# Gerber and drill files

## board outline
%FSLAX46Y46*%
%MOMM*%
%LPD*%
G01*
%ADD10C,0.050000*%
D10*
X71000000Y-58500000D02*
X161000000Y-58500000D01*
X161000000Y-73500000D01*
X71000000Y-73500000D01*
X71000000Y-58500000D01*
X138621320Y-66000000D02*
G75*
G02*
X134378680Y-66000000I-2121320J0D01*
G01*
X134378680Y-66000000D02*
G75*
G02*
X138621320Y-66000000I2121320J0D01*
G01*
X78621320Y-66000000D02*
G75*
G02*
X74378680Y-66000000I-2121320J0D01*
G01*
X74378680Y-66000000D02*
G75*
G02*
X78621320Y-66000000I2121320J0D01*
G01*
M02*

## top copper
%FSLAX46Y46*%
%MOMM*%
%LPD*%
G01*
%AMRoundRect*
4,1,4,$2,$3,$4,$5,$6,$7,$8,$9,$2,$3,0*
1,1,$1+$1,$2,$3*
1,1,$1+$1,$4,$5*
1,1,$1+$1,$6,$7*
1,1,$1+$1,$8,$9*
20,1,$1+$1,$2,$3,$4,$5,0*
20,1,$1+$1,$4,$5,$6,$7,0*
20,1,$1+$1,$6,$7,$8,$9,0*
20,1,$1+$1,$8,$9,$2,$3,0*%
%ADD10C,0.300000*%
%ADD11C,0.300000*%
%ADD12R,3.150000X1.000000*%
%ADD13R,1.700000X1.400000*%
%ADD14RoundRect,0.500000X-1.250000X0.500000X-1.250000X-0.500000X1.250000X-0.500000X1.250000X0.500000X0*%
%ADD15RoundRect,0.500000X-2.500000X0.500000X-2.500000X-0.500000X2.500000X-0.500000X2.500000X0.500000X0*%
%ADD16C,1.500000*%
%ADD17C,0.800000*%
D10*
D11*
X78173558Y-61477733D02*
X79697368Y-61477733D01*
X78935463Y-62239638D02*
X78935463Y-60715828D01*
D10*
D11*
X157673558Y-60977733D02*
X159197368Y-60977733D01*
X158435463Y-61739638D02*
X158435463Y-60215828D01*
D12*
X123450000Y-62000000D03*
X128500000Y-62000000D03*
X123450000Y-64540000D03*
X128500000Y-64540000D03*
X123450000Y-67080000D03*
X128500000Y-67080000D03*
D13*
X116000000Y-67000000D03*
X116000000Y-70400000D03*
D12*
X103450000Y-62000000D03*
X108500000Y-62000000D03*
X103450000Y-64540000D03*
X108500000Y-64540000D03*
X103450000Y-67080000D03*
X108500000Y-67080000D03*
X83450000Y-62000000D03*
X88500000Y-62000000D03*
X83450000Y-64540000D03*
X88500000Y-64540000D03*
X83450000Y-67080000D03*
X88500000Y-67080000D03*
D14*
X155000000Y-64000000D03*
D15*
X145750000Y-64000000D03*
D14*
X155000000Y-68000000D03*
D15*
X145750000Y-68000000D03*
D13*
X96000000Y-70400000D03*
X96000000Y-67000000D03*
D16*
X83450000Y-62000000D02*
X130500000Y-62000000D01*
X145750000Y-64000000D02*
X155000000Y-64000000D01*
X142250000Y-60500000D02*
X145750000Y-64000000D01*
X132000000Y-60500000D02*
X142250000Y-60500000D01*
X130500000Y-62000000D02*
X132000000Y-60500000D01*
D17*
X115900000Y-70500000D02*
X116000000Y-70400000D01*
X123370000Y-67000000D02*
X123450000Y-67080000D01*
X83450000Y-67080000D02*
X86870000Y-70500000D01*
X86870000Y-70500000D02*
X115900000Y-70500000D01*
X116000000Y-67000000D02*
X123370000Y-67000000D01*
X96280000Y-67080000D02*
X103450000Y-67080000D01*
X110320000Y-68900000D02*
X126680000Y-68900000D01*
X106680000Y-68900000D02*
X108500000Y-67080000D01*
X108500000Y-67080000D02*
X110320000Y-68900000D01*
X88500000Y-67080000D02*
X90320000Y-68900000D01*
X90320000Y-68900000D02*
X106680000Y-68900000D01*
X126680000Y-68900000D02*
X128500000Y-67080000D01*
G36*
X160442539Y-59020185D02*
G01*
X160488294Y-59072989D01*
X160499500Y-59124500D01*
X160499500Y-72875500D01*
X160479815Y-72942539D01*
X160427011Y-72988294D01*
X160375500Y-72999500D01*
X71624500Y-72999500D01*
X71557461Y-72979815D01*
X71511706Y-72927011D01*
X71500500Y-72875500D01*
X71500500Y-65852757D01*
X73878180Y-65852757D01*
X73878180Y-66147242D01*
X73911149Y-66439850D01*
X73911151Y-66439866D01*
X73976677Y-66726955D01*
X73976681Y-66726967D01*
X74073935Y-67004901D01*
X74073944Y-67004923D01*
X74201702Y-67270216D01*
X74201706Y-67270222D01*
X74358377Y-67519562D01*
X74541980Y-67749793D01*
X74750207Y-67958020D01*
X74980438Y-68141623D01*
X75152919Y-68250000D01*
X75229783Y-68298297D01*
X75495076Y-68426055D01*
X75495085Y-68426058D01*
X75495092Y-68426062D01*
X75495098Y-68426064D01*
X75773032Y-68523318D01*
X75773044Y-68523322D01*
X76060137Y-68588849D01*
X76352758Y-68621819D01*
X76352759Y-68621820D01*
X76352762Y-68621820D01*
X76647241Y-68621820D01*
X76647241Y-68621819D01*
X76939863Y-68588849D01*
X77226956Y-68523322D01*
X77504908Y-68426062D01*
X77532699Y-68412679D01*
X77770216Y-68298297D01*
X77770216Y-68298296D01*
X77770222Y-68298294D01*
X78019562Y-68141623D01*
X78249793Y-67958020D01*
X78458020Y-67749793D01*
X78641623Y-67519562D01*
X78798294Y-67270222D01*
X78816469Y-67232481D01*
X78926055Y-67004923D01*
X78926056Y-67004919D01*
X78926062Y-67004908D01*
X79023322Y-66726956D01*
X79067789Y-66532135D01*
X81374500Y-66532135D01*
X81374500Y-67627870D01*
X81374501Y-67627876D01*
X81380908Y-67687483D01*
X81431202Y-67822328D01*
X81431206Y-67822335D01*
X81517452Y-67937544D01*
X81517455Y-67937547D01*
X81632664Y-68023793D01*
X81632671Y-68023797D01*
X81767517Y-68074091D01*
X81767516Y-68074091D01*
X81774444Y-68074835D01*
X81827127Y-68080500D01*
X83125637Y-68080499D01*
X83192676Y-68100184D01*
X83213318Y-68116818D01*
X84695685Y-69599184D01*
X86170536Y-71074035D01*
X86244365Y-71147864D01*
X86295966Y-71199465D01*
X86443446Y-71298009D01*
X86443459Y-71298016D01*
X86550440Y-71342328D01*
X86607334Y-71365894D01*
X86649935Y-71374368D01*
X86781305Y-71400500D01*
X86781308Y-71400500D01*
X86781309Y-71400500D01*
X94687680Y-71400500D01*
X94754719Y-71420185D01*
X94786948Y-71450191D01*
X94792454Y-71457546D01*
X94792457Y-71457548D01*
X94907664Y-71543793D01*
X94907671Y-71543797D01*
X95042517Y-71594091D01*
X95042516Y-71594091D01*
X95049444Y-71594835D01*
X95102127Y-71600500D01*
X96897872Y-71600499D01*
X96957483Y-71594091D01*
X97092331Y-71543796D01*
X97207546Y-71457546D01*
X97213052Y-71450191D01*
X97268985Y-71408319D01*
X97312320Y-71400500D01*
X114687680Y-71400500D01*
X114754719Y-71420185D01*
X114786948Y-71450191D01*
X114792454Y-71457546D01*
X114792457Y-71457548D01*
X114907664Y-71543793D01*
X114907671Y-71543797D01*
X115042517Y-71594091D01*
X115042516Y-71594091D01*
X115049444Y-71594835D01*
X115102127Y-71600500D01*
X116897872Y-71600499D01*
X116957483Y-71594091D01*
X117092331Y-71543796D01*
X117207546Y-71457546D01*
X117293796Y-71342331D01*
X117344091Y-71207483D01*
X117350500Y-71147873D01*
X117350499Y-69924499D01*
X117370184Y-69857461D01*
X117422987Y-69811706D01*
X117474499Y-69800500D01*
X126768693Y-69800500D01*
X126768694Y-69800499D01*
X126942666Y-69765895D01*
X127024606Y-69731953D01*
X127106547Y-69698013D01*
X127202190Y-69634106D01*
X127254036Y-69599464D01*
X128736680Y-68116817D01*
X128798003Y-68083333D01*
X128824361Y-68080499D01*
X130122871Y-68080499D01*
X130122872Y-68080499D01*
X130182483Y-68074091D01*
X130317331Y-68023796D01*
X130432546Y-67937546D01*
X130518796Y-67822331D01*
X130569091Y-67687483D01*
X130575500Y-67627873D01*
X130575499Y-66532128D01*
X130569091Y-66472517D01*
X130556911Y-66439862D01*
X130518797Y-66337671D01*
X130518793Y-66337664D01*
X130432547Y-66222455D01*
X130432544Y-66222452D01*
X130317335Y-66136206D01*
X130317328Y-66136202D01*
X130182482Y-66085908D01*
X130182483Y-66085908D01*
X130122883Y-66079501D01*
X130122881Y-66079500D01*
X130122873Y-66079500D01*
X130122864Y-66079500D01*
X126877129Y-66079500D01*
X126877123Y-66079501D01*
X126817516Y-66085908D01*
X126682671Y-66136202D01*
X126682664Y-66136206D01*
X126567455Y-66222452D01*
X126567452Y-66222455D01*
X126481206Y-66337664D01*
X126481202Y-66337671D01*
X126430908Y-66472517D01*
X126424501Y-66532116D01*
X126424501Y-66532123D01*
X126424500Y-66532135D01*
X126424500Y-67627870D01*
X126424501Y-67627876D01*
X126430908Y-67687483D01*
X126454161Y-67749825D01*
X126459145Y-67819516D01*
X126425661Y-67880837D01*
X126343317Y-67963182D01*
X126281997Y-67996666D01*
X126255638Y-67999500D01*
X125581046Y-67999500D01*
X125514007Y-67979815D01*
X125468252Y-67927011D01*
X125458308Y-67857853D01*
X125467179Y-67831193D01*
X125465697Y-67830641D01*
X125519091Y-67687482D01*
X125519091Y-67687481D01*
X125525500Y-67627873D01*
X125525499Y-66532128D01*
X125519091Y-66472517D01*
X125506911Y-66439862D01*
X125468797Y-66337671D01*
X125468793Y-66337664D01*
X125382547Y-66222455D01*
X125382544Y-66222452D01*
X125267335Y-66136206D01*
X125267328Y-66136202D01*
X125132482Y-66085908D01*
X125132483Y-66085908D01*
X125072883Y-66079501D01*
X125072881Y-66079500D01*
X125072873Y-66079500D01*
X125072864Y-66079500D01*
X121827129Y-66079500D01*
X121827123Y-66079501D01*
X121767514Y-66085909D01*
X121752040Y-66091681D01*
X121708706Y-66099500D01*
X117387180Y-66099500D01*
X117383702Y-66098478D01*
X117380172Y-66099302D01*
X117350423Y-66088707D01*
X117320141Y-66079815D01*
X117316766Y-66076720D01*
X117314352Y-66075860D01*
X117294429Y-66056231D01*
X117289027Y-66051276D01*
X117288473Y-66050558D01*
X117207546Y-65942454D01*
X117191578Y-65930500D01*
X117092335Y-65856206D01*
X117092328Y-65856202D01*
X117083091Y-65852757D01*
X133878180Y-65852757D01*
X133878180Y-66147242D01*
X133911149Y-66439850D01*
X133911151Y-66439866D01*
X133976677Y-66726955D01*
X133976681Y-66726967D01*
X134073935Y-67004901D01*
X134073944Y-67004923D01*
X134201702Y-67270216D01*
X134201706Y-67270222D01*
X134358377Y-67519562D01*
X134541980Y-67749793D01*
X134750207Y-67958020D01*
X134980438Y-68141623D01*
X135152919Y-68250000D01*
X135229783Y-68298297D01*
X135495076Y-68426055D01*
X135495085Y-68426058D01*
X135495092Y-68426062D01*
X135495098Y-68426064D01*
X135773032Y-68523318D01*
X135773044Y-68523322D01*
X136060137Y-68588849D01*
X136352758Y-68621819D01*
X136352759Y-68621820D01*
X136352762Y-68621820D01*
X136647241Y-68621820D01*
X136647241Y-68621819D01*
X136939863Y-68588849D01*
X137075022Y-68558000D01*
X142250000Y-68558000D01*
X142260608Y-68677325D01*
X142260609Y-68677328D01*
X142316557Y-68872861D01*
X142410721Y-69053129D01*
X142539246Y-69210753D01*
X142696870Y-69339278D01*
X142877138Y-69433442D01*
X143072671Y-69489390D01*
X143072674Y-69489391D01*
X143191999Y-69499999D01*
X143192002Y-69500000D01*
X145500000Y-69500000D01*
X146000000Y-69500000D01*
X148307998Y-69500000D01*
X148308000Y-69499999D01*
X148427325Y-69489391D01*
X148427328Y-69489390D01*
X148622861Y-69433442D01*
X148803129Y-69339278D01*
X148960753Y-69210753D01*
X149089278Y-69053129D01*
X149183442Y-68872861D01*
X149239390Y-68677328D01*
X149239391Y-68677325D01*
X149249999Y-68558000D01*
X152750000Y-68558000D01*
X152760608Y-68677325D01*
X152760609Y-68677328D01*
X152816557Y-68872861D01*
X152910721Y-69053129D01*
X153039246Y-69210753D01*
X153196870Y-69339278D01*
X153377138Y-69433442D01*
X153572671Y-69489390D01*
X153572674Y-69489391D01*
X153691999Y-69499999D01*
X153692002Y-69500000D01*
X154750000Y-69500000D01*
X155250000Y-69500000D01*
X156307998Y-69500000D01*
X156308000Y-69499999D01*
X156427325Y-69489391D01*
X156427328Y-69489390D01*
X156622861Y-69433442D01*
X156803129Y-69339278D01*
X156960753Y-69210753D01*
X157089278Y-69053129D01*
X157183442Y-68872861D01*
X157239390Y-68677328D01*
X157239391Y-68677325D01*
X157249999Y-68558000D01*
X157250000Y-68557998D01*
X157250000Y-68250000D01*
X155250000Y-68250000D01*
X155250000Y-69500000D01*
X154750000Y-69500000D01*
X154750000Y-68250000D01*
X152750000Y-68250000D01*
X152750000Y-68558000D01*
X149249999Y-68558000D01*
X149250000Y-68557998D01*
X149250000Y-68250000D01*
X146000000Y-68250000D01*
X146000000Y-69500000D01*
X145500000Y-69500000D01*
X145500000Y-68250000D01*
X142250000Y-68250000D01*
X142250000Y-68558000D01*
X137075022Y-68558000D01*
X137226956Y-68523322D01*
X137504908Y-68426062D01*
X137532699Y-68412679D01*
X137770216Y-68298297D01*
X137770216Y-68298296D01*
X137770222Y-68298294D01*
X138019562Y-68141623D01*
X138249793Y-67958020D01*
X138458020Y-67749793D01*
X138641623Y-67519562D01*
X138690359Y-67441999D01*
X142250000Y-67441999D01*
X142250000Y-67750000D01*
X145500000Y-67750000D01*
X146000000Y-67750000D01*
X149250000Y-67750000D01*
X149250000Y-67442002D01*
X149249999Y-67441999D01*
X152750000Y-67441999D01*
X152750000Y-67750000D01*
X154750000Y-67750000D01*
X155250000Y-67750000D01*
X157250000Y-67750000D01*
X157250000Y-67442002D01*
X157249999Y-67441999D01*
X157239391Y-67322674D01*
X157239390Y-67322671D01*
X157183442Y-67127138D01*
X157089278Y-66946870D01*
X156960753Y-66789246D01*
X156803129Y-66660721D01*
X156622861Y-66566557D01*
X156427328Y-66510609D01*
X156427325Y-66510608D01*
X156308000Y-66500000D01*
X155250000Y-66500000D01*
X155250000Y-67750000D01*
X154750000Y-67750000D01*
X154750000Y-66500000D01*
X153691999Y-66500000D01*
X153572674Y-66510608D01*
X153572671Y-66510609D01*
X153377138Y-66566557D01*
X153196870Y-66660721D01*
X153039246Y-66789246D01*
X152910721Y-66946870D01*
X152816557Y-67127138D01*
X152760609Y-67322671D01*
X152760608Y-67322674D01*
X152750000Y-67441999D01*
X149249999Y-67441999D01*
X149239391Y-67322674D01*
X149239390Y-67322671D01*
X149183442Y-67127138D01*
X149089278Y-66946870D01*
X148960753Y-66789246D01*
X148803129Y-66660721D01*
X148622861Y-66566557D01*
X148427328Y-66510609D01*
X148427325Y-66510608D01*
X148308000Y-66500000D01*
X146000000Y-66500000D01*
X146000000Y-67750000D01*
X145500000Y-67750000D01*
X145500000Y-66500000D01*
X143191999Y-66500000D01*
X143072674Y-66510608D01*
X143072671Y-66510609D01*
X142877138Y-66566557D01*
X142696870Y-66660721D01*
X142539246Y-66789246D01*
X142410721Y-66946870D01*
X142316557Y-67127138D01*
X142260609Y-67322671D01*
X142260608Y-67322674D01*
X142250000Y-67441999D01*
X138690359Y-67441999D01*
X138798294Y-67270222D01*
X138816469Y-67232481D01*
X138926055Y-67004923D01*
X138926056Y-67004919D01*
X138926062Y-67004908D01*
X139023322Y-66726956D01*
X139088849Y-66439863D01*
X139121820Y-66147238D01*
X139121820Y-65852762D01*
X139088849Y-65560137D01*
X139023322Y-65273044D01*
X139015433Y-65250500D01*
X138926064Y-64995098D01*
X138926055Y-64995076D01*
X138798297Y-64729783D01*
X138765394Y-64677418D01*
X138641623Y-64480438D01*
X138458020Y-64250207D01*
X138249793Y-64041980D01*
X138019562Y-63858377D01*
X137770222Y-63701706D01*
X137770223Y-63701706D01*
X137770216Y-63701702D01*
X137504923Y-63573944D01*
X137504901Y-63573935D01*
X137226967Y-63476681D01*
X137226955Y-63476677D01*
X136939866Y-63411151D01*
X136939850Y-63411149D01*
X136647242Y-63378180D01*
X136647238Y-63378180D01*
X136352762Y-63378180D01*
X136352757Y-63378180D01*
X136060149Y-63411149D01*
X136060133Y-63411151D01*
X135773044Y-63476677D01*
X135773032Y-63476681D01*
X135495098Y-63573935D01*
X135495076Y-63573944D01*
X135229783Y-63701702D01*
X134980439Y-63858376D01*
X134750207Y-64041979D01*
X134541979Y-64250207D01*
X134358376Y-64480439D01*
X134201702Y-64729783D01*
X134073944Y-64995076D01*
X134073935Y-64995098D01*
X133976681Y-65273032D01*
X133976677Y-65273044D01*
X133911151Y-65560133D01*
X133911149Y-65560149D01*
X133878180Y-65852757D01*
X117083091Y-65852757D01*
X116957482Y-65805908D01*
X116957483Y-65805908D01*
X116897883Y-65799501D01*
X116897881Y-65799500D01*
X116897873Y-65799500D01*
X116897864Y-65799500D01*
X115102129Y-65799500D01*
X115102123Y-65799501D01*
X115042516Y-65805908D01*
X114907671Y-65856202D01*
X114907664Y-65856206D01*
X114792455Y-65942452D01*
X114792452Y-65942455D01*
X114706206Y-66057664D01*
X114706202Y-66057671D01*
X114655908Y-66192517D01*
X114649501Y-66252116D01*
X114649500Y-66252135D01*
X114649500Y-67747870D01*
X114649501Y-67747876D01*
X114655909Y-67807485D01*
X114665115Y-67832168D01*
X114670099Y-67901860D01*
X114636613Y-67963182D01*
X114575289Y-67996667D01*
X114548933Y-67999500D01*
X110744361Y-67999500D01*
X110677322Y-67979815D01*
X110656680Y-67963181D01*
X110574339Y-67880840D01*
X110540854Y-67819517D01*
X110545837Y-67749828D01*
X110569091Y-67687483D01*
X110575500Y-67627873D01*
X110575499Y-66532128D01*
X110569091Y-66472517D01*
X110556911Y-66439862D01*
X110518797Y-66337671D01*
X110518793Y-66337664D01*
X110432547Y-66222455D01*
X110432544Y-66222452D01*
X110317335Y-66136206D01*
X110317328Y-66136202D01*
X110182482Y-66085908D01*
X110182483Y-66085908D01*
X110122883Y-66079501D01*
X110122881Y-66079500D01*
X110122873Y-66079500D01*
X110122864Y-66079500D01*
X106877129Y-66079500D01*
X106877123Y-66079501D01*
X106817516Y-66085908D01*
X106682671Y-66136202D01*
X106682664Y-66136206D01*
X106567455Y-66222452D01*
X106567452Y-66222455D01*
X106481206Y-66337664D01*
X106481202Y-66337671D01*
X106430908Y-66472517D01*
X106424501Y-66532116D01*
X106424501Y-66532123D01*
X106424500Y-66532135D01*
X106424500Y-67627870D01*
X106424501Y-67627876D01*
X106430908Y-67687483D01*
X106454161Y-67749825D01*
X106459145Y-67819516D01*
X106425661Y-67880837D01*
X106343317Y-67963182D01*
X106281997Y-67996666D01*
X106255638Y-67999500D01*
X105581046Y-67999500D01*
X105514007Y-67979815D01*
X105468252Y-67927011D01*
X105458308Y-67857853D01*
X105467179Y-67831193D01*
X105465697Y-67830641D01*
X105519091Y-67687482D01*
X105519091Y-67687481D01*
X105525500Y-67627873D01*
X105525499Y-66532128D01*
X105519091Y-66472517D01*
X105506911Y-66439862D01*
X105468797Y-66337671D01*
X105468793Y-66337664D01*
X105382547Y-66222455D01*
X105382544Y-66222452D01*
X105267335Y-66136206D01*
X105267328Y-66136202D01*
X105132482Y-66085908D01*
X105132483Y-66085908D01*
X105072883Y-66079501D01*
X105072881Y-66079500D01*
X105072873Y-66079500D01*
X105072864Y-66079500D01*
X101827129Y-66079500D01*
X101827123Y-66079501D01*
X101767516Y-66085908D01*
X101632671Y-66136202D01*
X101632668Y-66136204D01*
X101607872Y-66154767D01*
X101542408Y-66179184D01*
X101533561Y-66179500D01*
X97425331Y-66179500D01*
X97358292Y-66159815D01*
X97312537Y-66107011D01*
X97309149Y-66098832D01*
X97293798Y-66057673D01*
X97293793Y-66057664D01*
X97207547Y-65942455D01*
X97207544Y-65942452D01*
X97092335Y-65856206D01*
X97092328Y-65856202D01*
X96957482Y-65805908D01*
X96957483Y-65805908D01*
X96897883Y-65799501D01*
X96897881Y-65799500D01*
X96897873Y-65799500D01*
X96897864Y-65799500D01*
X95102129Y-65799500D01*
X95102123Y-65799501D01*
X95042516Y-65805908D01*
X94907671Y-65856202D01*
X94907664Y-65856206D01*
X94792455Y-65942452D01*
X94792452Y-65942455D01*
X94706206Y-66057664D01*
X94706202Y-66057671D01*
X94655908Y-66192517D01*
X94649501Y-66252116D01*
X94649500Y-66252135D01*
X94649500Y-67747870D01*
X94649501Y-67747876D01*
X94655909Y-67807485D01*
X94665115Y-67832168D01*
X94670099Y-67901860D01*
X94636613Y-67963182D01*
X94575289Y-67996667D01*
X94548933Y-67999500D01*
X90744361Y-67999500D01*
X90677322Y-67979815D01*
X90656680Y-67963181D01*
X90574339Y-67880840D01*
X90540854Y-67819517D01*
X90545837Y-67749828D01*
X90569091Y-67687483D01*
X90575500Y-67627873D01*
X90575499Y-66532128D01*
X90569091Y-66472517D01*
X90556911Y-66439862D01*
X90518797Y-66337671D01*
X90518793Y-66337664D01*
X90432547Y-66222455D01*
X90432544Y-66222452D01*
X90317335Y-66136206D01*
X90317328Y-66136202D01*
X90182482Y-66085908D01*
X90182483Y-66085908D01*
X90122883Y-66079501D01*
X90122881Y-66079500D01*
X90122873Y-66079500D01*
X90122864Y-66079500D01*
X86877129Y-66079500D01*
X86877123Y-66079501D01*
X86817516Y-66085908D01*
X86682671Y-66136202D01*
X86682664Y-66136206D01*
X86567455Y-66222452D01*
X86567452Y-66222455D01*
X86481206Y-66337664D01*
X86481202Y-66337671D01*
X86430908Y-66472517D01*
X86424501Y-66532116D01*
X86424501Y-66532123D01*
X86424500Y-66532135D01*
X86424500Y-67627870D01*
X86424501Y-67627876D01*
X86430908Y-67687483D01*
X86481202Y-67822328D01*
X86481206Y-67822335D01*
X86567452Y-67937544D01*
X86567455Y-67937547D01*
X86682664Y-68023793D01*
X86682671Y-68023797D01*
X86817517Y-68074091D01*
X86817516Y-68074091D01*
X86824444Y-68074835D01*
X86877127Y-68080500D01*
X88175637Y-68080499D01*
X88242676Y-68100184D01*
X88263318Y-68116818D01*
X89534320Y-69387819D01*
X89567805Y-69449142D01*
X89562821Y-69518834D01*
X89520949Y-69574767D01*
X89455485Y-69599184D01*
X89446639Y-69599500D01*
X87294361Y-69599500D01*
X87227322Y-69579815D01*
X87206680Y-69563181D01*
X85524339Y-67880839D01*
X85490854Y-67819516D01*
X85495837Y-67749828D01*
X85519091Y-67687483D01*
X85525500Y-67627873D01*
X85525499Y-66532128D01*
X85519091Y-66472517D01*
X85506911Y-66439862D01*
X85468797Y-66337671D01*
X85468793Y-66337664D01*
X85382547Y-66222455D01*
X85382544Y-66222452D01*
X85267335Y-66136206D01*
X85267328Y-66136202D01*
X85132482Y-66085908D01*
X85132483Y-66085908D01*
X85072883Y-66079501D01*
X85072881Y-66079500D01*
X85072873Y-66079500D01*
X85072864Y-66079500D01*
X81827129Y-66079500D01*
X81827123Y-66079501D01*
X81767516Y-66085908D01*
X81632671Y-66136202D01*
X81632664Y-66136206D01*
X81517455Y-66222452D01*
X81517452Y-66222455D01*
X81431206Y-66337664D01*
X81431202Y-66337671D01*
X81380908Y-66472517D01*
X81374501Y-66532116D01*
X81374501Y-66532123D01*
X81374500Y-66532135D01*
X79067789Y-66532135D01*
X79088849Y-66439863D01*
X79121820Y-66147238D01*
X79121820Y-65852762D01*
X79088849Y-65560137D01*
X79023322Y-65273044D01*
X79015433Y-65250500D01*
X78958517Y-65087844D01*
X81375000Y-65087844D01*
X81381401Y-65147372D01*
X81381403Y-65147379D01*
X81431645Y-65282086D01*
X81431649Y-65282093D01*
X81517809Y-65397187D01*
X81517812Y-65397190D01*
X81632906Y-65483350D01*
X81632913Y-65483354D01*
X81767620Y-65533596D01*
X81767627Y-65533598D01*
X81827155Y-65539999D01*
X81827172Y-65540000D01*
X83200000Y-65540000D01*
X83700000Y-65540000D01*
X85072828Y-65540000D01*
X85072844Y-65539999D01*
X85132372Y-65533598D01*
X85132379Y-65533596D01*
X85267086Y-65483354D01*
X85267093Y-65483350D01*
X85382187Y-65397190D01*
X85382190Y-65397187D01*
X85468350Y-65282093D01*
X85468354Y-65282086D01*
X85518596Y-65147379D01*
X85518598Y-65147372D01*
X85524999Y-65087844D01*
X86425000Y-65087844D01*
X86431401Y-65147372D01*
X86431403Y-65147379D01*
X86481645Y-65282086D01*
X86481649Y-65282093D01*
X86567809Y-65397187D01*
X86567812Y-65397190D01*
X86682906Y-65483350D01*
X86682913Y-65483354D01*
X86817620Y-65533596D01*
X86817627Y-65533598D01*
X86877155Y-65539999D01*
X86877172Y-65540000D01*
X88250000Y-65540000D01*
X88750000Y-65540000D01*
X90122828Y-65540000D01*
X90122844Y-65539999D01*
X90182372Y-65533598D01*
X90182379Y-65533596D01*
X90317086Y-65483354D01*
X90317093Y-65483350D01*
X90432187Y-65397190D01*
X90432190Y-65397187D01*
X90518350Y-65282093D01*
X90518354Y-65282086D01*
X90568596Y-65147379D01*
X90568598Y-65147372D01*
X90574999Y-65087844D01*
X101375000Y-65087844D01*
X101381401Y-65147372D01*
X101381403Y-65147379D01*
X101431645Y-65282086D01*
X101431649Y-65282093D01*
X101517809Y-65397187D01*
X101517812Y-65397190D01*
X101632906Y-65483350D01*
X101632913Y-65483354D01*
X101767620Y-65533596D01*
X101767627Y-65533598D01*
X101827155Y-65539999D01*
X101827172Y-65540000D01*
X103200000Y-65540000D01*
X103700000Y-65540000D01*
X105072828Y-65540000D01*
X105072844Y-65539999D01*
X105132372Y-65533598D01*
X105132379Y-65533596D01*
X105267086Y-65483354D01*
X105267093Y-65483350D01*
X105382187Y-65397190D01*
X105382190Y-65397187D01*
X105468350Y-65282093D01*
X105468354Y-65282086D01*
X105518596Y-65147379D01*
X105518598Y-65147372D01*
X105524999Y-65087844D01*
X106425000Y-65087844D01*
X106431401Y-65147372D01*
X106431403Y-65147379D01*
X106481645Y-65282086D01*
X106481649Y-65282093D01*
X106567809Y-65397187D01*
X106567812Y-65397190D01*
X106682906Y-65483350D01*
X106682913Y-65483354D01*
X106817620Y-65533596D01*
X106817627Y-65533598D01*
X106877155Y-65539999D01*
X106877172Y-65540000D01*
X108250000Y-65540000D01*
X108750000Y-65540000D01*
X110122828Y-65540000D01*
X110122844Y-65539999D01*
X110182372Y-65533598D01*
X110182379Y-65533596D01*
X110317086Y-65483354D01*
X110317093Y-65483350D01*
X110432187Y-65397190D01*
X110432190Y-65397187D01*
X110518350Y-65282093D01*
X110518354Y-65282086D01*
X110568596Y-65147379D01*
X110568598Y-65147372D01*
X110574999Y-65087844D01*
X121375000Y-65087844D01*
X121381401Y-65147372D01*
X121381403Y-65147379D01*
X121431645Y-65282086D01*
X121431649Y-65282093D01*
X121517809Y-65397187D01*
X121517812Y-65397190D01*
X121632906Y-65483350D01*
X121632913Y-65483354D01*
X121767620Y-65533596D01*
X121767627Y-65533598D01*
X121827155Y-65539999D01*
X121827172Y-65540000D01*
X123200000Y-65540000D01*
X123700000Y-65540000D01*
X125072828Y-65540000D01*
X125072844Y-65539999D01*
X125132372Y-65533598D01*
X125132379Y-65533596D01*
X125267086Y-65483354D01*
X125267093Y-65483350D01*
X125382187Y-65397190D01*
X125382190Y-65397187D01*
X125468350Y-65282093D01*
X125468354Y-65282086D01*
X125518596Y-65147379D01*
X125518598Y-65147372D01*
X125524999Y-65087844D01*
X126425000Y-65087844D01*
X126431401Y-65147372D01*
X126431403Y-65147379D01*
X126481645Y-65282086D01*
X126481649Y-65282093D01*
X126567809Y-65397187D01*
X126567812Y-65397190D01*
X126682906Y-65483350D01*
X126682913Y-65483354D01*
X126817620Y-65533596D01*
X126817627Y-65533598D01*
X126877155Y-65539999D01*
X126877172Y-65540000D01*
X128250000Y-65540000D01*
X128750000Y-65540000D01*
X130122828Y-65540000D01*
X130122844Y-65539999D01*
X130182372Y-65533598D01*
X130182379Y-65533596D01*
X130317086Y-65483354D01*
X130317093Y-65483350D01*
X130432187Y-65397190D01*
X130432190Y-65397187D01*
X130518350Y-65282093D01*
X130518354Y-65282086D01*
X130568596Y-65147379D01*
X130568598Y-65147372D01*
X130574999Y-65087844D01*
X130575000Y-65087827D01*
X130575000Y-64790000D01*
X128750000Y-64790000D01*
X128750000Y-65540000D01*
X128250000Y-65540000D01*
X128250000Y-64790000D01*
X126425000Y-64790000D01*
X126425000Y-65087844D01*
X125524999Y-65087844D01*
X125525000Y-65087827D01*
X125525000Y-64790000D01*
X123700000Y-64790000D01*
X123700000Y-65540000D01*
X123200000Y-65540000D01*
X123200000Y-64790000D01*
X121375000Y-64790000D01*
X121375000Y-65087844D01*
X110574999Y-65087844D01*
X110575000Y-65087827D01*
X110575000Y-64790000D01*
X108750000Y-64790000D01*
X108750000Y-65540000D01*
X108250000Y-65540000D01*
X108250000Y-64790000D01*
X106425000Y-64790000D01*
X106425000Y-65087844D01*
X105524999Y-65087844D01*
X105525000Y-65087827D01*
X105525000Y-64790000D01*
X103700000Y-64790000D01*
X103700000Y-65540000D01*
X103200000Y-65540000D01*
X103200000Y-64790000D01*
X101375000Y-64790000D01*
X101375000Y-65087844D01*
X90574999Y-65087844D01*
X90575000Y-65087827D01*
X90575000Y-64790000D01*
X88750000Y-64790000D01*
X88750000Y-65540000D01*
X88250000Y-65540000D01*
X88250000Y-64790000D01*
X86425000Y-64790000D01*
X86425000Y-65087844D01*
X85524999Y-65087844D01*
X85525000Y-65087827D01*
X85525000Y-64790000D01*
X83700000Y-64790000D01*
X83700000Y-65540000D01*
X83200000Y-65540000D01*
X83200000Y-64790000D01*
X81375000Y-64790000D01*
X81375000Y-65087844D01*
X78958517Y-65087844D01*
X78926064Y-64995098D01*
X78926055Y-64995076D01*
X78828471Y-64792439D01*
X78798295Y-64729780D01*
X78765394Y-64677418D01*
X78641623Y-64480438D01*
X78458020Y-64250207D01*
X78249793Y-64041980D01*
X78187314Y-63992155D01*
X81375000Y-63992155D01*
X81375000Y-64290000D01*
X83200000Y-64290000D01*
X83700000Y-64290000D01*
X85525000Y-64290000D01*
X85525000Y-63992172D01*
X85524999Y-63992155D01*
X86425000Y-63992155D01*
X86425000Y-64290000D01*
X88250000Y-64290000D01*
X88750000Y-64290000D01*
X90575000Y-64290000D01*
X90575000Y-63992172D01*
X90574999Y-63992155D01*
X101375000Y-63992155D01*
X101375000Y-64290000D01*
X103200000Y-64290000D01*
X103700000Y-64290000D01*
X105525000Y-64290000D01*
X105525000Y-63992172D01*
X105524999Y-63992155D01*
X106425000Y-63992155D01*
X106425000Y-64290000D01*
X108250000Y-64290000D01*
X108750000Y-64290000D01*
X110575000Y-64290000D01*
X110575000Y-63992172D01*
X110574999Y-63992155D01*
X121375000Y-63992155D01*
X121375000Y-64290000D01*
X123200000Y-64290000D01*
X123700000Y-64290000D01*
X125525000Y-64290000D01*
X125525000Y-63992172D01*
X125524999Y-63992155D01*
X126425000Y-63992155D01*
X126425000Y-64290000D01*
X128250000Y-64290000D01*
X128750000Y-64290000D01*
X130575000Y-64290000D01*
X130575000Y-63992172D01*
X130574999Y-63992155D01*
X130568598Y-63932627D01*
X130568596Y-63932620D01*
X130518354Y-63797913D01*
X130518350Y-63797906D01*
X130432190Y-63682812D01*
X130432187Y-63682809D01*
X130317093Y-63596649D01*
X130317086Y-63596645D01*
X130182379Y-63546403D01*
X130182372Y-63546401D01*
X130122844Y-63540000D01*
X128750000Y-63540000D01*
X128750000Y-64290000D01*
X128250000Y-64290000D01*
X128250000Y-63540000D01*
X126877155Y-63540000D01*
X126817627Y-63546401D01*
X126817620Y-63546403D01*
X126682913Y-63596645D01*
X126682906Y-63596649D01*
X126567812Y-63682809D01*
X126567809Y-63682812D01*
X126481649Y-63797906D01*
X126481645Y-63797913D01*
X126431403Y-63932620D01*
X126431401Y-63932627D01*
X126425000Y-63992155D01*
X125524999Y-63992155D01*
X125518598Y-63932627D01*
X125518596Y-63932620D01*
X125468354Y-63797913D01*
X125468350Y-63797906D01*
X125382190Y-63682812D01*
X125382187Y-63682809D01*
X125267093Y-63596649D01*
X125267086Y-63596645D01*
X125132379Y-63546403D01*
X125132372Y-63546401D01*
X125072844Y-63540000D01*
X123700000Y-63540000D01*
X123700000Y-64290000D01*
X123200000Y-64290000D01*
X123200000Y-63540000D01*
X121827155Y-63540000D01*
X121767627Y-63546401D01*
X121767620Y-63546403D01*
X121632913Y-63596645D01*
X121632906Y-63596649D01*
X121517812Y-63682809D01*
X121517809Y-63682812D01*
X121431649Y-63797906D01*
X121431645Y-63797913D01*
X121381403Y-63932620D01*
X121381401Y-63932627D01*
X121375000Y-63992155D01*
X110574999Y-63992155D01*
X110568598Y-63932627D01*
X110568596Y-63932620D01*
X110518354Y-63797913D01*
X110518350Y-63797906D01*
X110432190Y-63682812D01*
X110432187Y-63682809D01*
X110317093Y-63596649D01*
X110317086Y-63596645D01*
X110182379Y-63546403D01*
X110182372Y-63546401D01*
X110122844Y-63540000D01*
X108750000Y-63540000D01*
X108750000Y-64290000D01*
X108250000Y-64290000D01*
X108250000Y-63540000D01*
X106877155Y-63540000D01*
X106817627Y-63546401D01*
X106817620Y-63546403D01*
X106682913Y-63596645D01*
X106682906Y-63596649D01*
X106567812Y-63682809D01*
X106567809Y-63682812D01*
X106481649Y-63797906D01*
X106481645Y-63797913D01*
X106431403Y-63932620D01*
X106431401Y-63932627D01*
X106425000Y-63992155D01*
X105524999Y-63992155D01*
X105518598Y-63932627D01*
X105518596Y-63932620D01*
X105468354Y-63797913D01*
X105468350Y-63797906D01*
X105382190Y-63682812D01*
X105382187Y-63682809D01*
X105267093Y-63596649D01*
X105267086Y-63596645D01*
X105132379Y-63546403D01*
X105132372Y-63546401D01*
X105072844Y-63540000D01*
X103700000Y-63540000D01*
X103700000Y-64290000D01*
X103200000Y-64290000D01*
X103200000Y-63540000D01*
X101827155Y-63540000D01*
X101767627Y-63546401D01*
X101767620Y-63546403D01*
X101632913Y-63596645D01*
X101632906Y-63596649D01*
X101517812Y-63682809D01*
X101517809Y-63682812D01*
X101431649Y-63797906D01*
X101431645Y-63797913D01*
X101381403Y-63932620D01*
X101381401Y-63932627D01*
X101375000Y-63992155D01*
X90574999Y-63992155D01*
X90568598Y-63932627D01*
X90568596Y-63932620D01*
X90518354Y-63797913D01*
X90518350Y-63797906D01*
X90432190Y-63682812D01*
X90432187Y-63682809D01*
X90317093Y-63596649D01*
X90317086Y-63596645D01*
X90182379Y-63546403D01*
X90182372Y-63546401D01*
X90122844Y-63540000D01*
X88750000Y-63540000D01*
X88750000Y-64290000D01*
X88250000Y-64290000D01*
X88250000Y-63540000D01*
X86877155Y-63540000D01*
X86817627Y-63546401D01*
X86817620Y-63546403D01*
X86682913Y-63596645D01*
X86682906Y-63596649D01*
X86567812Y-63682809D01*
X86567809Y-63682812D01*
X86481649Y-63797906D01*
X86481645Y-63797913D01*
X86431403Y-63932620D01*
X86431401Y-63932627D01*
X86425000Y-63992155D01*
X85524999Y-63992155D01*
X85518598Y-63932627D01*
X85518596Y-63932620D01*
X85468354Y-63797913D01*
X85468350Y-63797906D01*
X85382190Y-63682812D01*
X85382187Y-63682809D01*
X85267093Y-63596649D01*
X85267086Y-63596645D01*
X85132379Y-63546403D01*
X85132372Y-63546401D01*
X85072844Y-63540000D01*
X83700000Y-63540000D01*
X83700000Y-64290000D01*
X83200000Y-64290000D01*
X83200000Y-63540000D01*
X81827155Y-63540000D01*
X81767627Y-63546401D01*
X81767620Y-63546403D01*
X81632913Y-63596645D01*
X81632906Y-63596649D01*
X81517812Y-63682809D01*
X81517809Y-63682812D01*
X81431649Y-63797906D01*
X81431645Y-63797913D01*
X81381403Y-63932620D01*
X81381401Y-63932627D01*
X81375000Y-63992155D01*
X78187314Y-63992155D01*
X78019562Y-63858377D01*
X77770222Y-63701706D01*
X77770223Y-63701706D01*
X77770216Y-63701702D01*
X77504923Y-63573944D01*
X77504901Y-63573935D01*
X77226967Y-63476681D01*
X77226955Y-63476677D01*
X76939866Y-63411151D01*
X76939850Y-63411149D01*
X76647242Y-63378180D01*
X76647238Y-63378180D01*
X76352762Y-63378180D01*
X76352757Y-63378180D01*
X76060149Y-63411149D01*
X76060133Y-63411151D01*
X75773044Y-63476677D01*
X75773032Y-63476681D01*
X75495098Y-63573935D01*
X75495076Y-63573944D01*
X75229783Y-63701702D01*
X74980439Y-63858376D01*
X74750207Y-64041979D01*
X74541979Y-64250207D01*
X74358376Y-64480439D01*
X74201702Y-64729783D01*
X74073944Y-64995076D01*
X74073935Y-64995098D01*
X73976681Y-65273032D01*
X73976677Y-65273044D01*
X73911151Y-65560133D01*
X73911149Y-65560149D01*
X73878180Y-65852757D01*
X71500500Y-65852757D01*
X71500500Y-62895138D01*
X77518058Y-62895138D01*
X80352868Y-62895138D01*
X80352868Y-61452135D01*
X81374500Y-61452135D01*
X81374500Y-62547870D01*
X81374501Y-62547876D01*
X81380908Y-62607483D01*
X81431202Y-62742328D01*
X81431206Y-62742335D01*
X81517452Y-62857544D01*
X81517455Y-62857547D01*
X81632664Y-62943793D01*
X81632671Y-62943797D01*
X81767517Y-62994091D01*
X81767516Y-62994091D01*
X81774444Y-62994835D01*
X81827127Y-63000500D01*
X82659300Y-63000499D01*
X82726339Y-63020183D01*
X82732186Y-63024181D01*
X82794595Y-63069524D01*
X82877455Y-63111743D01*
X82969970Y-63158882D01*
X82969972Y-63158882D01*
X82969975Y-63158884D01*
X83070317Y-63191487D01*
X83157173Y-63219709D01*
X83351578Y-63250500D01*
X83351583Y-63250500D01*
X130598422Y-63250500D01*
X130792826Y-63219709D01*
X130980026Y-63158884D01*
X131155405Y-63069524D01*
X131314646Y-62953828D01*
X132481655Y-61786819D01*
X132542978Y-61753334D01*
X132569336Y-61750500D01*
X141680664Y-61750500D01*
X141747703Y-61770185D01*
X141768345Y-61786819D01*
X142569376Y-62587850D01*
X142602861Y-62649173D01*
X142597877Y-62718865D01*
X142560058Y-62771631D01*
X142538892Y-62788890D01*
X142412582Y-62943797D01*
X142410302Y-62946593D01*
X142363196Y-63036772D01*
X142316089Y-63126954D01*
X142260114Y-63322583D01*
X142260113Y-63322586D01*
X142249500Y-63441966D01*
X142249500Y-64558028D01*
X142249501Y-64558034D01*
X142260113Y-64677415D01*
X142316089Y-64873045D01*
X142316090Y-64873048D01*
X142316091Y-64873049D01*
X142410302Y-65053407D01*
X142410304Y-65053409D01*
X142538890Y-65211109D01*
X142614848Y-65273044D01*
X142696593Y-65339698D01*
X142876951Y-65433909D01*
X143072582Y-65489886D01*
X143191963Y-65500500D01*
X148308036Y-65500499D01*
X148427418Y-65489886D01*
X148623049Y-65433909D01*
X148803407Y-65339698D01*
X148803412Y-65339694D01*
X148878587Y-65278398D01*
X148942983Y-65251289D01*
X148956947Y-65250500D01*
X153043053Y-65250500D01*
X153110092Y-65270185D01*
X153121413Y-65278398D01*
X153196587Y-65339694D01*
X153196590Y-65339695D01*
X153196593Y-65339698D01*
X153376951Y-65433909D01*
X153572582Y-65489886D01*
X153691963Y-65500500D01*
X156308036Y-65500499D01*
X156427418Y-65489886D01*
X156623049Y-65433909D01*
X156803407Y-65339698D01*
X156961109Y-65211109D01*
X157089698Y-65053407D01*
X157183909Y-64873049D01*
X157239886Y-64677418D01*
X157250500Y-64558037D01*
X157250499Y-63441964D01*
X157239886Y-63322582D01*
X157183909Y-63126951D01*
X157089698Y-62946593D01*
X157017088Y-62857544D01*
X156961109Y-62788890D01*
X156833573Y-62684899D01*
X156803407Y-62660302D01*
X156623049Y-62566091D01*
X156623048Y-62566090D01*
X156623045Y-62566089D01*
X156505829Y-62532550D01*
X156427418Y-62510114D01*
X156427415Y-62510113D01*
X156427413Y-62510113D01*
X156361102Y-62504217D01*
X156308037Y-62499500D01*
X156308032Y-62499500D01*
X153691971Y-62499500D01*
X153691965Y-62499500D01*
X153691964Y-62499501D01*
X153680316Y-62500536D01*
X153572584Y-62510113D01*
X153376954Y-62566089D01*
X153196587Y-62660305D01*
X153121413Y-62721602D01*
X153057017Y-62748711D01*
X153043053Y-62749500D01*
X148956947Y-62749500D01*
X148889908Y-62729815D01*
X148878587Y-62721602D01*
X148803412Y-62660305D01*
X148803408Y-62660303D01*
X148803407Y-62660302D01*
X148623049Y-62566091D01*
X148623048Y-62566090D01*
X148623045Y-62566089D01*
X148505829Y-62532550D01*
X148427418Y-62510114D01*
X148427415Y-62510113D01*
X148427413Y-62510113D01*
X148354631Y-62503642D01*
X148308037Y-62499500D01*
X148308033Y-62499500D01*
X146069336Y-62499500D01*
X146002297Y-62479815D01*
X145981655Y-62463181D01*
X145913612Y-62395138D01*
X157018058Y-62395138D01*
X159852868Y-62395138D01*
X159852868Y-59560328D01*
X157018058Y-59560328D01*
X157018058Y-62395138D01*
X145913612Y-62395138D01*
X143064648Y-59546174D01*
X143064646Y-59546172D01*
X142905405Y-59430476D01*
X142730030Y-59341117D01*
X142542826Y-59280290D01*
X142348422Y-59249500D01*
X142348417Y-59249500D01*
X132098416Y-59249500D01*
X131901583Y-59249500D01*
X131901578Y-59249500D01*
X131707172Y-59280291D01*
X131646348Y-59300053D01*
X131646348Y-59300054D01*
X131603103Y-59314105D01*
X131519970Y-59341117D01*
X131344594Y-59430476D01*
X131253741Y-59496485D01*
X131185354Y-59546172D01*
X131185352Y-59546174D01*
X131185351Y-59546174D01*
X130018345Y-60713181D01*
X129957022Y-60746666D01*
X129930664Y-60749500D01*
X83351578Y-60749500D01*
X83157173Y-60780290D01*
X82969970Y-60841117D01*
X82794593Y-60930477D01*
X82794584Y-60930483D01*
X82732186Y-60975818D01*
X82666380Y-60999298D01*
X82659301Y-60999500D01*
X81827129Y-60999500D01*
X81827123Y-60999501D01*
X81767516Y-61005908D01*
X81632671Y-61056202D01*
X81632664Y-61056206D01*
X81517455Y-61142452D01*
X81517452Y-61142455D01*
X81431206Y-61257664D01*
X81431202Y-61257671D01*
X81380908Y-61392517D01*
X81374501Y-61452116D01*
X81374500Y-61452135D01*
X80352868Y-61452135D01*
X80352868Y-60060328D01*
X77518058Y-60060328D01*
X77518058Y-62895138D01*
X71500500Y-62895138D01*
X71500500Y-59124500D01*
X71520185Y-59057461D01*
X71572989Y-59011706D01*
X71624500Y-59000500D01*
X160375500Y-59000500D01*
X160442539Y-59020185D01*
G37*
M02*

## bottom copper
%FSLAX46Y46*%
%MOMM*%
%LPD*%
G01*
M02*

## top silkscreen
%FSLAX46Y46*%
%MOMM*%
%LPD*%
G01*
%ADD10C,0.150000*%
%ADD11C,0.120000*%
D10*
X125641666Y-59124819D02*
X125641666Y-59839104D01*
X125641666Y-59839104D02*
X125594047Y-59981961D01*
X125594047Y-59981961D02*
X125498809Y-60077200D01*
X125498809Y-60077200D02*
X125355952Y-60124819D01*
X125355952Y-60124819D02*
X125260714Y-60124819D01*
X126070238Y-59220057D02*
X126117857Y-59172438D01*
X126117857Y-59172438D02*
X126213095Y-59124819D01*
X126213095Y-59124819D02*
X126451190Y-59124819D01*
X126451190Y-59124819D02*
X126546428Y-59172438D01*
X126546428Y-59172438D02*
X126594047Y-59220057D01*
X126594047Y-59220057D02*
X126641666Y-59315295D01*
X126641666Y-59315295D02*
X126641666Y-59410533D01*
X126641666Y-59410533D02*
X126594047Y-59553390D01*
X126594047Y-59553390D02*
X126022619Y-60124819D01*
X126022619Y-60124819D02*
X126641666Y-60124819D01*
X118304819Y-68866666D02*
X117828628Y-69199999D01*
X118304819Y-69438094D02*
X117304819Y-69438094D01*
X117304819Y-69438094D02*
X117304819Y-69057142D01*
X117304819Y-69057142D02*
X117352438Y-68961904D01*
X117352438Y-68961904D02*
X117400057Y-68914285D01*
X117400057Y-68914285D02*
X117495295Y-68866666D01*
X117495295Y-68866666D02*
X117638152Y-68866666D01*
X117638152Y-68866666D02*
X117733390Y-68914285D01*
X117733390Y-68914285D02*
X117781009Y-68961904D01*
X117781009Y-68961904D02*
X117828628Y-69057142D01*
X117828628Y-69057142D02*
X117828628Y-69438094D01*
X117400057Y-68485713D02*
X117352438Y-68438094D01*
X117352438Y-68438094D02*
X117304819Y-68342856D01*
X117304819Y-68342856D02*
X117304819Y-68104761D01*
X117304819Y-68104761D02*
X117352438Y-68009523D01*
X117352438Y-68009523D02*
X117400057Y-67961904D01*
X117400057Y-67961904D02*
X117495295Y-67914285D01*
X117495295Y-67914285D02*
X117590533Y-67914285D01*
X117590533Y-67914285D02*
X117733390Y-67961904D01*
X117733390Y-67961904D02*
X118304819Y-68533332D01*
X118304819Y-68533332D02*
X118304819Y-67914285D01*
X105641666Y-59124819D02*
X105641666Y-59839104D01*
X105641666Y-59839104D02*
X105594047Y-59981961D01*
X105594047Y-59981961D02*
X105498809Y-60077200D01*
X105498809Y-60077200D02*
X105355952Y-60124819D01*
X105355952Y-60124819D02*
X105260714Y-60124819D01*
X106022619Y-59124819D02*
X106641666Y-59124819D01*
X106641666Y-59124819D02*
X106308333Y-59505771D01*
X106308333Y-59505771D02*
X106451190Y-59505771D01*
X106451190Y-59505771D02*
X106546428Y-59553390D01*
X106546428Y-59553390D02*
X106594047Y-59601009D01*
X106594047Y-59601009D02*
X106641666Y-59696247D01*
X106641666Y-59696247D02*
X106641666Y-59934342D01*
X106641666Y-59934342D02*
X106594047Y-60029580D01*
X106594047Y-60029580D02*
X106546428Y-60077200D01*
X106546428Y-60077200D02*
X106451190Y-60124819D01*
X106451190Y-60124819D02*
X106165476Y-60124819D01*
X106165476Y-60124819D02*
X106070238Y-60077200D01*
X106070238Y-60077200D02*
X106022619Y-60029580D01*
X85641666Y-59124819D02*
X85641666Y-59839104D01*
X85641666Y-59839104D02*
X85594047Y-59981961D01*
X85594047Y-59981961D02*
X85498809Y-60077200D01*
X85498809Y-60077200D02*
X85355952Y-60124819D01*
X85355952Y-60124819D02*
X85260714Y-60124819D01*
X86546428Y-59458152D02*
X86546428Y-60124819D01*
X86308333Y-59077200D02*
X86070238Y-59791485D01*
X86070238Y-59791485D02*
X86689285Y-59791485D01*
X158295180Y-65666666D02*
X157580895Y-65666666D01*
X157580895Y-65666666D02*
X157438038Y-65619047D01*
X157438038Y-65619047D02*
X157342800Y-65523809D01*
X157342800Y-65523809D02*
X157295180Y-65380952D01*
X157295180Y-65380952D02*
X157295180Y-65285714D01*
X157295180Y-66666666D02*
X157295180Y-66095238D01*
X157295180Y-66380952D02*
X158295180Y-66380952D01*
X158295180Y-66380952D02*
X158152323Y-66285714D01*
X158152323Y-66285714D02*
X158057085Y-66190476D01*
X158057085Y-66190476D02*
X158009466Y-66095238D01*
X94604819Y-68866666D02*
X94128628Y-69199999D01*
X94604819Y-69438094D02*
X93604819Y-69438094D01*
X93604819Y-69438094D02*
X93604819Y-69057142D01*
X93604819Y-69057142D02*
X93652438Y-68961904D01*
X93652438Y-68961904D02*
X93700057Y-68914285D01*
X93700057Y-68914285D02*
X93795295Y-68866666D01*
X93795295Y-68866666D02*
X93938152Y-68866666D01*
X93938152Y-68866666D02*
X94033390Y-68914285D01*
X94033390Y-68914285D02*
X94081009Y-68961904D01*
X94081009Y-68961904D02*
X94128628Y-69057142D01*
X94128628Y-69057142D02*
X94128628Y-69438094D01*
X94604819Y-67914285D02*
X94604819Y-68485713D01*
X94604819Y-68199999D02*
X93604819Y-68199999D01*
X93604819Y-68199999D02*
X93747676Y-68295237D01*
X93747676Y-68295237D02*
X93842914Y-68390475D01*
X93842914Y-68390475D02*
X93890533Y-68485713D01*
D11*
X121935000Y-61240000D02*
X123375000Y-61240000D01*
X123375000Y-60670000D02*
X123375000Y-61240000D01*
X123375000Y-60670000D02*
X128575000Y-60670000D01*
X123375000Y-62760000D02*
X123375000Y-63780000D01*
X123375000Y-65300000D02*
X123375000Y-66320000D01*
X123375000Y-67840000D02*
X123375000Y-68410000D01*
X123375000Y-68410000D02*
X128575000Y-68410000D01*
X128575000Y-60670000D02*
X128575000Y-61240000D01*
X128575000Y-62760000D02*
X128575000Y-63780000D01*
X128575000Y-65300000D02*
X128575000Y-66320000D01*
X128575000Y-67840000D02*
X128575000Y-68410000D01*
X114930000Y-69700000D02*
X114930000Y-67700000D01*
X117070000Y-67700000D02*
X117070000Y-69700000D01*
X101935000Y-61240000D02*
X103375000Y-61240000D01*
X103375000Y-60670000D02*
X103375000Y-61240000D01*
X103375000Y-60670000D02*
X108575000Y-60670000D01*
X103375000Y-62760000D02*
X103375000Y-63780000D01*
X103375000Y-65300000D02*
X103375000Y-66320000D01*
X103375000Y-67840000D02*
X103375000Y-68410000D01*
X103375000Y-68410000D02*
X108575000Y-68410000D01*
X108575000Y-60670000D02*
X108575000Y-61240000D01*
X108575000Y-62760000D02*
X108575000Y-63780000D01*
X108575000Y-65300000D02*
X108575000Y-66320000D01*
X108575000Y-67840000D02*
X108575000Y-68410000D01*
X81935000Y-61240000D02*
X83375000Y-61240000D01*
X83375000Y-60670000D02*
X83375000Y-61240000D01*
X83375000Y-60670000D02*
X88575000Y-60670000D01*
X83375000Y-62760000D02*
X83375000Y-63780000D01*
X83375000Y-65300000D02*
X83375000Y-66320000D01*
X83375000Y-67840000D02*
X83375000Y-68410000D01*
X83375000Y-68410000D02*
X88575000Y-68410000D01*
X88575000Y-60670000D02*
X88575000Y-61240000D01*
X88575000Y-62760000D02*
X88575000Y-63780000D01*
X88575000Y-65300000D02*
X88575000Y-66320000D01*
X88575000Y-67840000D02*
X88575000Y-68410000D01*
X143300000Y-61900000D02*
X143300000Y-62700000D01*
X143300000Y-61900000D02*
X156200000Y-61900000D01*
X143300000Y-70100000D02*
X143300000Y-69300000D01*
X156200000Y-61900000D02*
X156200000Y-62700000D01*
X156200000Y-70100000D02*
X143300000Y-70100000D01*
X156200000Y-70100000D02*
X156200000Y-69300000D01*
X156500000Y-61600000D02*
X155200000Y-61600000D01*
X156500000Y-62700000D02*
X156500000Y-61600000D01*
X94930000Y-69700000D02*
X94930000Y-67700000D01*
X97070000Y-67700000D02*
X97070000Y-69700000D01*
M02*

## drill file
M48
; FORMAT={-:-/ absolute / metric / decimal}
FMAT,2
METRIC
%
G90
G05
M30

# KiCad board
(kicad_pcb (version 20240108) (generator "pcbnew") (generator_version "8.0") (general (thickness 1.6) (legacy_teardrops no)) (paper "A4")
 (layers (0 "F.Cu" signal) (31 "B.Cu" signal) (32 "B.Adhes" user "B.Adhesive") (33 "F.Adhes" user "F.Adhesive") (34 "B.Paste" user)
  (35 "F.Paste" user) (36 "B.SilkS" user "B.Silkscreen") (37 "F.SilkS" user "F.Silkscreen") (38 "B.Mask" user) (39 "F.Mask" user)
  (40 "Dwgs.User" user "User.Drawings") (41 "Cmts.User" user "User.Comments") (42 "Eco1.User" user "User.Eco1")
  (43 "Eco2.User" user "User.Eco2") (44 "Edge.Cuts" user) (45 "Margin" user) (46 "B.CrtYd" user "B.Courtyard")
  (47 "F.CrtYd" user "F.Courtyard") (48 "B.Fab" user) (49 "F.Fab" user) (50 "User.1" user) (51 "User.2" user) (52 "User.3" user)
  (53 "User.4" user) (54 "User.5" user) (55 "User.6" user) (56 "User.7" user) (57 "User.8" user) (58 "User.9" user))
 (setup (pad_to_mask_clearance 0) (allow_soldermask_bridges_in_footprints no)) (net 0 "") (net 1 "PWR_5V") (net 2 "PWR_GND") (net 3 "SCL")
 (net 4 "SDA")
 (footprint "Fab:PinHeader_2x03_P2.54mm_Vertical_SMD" (layer "F.Cu") (at 125.975 64.54)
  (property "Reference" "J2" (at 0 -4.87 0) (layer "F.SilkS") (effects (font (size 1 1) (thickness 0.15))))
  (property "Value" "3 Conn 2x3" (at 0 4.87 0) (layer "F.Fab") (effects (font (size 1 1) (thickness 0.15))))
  (fp_line (start -4.04 -3.3) (end -2.6 -3.3) (stroke (width 0.12) (type solid)) (layer "F.SilkS"))
  (fp_line (start -2.6 -3.87) (end -2.6 -3.3) (stroke (width 0.12) (type solid)) (layer "F.SilkS"))
  (fp_line (start -2.6 -3.87) (end 2.6 -3.87) (stroke (width 0.12) (type solid)) (layer "F.SilkS"))
  (fp_line (start -2.6 -1.78) (end -2.6 -0.76) (stroke (width 0.12) (type solid)) (layer "F.SilkS"))
  (fp_line (start -2.6 0.76) (end -2.6 1.78) (stroke (width 0.12) (type solid)) (layer "F.SilkS"))
  (fp_line (start -2.6 3.3) (end -2.6 3.87) (stroke (width 0.12) (type solid)) (layer "F.SilkS"))
  (fp_line (start -2.6 3.87) (end 2.6 3.87) (stroke (width 0.12) (type solid)) (layer "F.SilkS"))
  (fp_line (start 2.6 -3.87) (end 2.6 -3.3) (stroke (width 0.12) (type solid)) (layer "F.SilkS"))
  (fp_line (start 2.6 -1.78) (end 2.6 -0.76) (stroke (width 0.12) (type solid)) (layer "F.SilkS"))
  (fp_line (start 2.6 0.76) (end 2.6 1.78) (stroke (width 0.12) (type solid)) (layer "F.SilkS"))
  (fp_line (start 2.6 3.3) (end 2.6 3.87) (stroke (width 0.12) (type solid)) (layer "F.SilkS"))
  (pad "1" smd rect (at -2.525 -2.54) (size 3.15 1) (layers "F.Cu" "F.Paste" "F.Mask") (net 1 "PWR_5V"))
  (pad "2" smd rect (at 2.525 -2.54) (size 3.15 1) (layers "F.Cu" "F.Paste" "F.Mask") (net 1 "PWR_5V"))
  (pad "3" smd rect (at -2.525 0) (size 3.15 1) (layers "F.Cu" "F.Paste" "F.Mask") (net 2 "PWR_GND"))
  (pad "4" smd rect (at 2.525 0) (size 3.15 1) (layers "F.Cu" "F.Paste" "F.Mask") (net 2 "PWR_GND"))
  (pad "5" smd rect (at -2.525 2.54) (size 3.15 1) (layers "F.Cu" "F.Paste" "F.Mask") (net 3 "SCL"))
  (pad "6" smd rect (at 2.525 2.54) (size 3.15 1) (layers "F.Cu" "F.Paste" "F.Mask") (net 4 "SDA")))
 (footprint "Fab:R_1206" (layer "F.Cu") (at 116 68.7 -90)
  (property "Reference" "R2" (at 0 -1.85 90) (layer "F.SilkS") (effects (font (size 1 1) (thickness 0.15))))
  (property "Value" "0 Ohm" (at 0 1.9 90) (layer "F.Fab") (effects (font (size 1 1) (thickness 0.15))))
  (fp_line (start 1 1.07) (end -1 1.07) (stroke (width 0.12) (type solid)) (layer "F.SilkS"))
  (fp_line (start -1 -1.07) (end 1 -1.07) (stroke (width 0.12) (type solid)) (layer "F.SilkS"))
  (pad "1" smd rect (at -1.7 0 270) (size 1.4 1.7) (layers "F.Cu" "F.Paste" "F.Mask") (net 3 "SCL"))
  (pad "2" smd rect (at 1.7 0 270) (size 1.4 1.7) (layers "F.Cu" "F.Paste" "F.Mask") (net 3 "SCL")))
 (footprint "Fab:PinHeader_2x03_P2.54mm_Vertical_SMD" (layer "F.Cu") (at 105.975 64.54)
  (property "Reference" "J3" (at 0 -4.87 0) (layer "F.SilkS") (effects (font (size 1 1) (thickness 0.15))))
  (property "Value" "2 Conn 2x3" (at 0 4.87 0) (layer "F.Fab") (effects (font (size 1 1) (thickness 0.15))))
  (fp_line (start -4.04 -3.3) (end -2.6 -3.3) (stroke (width 0.12) (type solid)) (layer "F.SilkS"))
  (fp_line (start -2.6 -3.87) (end -2.6 -3.3) (stroke (width 0.12) (type solid)) (layer "F.SilkS"))
  (fp_line (start -2.6 -3.87) (end 2.6 -3.87) (stroke (width 0.12) (type solid)) (layer "F.SilkS"))
  (fp_line (start -2.6 -1.78) (end -2.6 -0.76) (stroke (width 0.12) (type solid)) (layer "F.SilkS"))
  (fp_line (start -2.6 0.76) (end -2.6 1.78) (stroke (width 0.12) (type solid)) (layer "F.SilkS"))
  (fp_line (start -2.6 3.3) (end -2.6 3.87) (stroke (width 0.12) (type solid)) (layer "F.SilkS"))
  (fp_line (start -2.6 3.87) (end 2.6 3.87) (stroke (width 0.12) (type solid)) (layer "F.SilkS"))
  (fp_line (start 2.6 -3.87) (end 2.6 -3.3) (stroke (width 0.12) (type solid)) (layer "F.SilkS"))
  (fp_line (start 2.6 -1.78) (end 2.6 -0.76) (stroke (width 0.12) (type solid)) (layer "F.SilkS"))
  (fp_line (start 2.6 0.76) (end 2.6 1.78) (stroke (width 0.12) (type solid)) (layer "F.SilkS"))
  (fp_line (start 2.6 3.3) (end 2.6 3.87) (stroke (width 0.12) (type solid)) (layer "F.SilkS"))
  (pad "1" smd rect (at -2.525 -2.54) (size 3.15 1) (layers "F.Cu" "F.Paste" "F.Mask") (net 1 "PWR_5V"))
  (pad "2" smd rect (at 2.525 -2.54) (size 3.15 1) (layers "F.Cu" "F.Paste" "F.Mask") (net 1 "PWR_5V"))
  (pad "3" smd rect (at -2.525 0) (size 3.15 1) (layers "F.Cu" "F.Paste" "F.Mask") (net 2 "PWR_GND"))
  (pad "4" smd rect (at 2.525 0) (size 3.15 1) (layers "F.Cu" "F.Paste" "F.Mask") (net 2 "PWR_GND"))
  (pad "5" smd rect (at -2.525 2.54) (size 3.15 1) (layers "F.Cu" "F.Paste" "F.Mask") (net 3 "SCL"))
  (pad "6" smd rect (at 2.525 2.54) (size 3.15 1) (layers "F.Cu" "F.Paste" "F.Mask") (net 4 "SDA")))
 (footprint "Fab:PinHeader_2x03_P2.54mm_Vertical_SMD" (layer "F.Cu") (at 85.975 64.54)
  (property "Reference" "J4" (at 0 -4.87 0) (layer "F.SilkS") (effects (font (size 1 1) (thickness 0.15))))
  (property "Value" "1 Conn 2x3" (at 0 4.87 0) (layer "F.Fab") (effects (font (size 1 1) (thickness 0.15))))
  (fp_line (start -4.04 -3.3) (end -2.6 -3.3) (stroke (width 0.12) (type solid)) (layer "F.SilkS"))
  (fp_line (start -2.6 -3.87) (end -2.6 -3.3) (stroke (width 0.12) (type solid)) (layer "F.SilkS"))
  (fp_line (start -2.6 -3.87) (end 2.6 -3.87) (stroke (width 0.12) (type solid)) (layer "F.SilkS"))
  (fp_line (start -2.6 -1.78) (end -2.6 -0.76) (stroke (width 0.12) (type solid)) (layer "F.SilkS"))
  (fp_line (start -2.6 0.76) (end -2.6 1.78) (stroke (width 0.12) (type solid)) (layer "F.SilkS"))
  (fp_line (start -2.6 3.3) (end -2.6 3.87) (stroke (width 0.12) (type solid)) (layer "F.SilkS"))
  (fp_line (start -2.6 3.87) (end 2.6 3.87) (stroke (width 0.12) (type solid)) (layer "F.SilkS"))
  (fp_line (start 2.6 -3.87) (end 2.6 -3.3) (stroke (width 0.12) (type solid)) (layer "F.SilkS"))
  (fp_line (start 2.6 -1.78) (end 2.6 -0.76) (stroke (width 0.12) (type solid)) (layer "F.SilkS"))
  (fp_line (start 2.6 0.76) (end 2.6 1.78) (stroke (width 0.12) (type solid)) (layer "F.SilkS"))
  (fp_line (start 2.6 3.3) (end 2.6 3.87) (stroke (width 0.12) (type solid)) (layer "F.SilkS"))
  (pad "1" smd rect (at -2.525 -2.54) (size 3.15 1) (layers "F.Cu" "F.Paste" "F.Mask") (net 1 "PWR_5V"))
  (pad "2" smd rect (at 2.525 -2.54) (size 3.15 1) (layers "F.Cu" "F.Paste" "F.Mask") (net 1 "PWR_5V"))
  (pad "3" smd rect (at -2.525 0) (size 3.15 1) (layers "F.Cu" "F.Paste" "F.Mask") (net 2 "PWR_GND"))
  (pad "4" smd rect (at 2.525 0) (size 3.15 1) (layers "F.Cu" "F.Paste" "F.Mask") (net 2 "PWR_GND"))
  (pad "5" smd rect (at -2.525 2.54) (size 3.15 1) (layers "F.Cu" "F.Paste" "F.Mask") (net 3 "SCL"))
  (pad "6" smd rect (at 2.525 2.54) (size 3.15 1) (layers "F.Cu" "F.Paste" "F.Mask") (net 4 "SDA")))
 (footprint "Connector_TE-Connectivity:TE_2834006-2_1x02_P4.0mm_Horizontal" (layer "F.Cu") (at 149.75 66 -90)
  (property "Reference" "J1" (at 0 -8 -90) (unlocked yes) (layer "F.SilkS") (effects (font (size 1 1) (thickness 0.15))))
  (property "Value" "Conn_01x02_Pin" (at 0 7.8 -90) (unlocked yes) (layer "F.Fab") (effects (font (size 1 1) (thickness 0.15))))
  (fp_line (start -4.1 6.45) (end -3.3 6.45) (stroke (width 0.12) (type solid)) (layer "F.SilkS"))
  (fp_line (start -4.1 6.45) (end -4.1 -6.45) (stroke (width 0.12) (type solid)) (layer "F.SilkS"))
  (fp_line (start 4.1 6.45) (end 3.3 6.45) (stroke (width 0.12) (type solid)) (layer "F.SilkS"))
  (fp_line (start -4.1 -6.45) (end -3.3 -6.45) (stroke (width 0.12) (type solid)) (layer "F.SilkS"))
  (fp_line (start 4.1 -6.45) (end 4.1 6.45) (stroke (width 0.12) (type solid)) (layer "F.SilkS"))
  (fp_line (start 4.1 -6.45) (end 3.3 -6.45) (stroke (width 0.12) (type solid)) (layer "F.SilkS"))
  (fp_line (start -4.4 -6.75) (end -4.4 -5.45) (stroke (width 0.12) (type solid)) (layer "F.SilkS"))
  (fp_line (start -3.3 -6.75) (end -4.4 -6.75) (stroke (width 0.12) (type solid)) (layer "F.SilkS"))
  (pad "1" smd roundrect (at -2 -5.25 270) (size 2 3.5) (layers "F.Cu" "F.Paste" "F.Mask") (roundrect_rratio 0.25) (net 1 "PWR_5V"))
  (pad "1" smd roundrect (at -2 4 270) (size 2 6) (layers "F.Cu" "F.Paste" "F.Mask") (roundrect_rratio 0.25) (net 1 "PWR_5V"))
  (pad "2" smd roundrect (at 2 -5.25 270) (size 2 3.5) (layers "F.Cu" "F.Paste" "F.Mask") (roundrect_rratio 0.25) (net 2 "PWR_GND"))
  (pad "2" smd roundrect (at 2 4 270) (size 2 6) (layers "F.Cu" "F.Paste" "F.Mask") (roundrect_rratio 0.25) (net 2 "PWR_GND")))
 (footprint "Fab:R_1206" (layer "F.Cu") (at 96 68.7 90)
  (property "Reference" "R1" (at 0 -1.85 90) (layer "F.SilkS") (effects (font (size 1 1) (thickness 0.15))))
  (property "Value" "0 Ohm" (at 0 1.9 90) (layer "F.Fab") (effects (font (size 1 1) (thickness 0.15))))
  (fp_line (start -1 -1.07) (end 1 -1.07) (stroke (width 0.12) (type solid)) (layer "F.SilkS"))
  (fp_line (start 1 1.07) (end -1 1.07) (stroke (width 0.12) (type solid)) (layer "F.SilkS"))
  (pad "1" smd rect (at -1.7 0 90) (size 1.4 1.7) (layers "F.Cu" "F.Paste" "F.Mask") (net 3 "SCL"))
  (pad "2" smd rect (at 1.7 0 90) (size 1.4 1.7) (layers "F.Cu" "F.Paste" "F.Mask") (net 3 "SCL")))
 (gr_rect (start 71 58.5) (end 161 73.5) (stroke (width 0.05) (type default)) (fill none) (layer "Edge.Cuts"))
 (gr_circle (center 136.5 66) (end 138 67.5) (stroke (width 0.05) (type default)) (fill none) (layer "Edge.Cuts"))
 (gr_circle (center 76.5 66) (end 78 67.5) (stroke (width 0.05) (type default)) (fill none) (layer "Edge.Cuts"))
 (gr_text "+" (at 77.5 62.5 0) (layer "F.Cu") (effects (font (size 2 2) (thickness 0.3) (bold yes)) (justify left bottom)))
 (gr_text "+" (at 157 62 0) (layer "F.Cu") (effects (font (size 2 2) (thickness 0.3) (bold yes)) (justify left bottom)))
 (segment (start 83.45 62) (end 130.5 62) (width 1.5) (layer "F.Cu") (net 1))
 (segment (start 145.75 64) (end 155 64) (width 1.5) (layer "F.Cu") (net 1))
 (segment (start 142.25 60.5) (end 145.75 64) (width 1.5) (layer "F.Cu") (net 1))
 (segment (start 132 60.5) (end 142.25 60.5) (width 1.5) (layer "F.Cu") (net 1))
 (segment (start 130.5 62) (end 132 60.5) (width 1.5) (layer "F.Cu") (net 1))
 (segment (start 115.9 70.5) (end 116 70.4) (width 0.8) (layer "F.Cu") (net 3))
 (segment (start 123.37 67) (end 123.45 67.08) (width 0.8) (layer "F.Cu") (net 3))
 (segment (start 83.45 67.08) (end 86.87 70.5) (width 0.8) (layer "F.Cu") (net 3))
 (segment (start 86.87 70.5) (end 115.9 70.5) (width 0.8) (layer "F.Cu") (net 3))
 (segment (start 116 67) (end 123.37 67) (width 0.8) (layer "F.Cu") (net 3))
 (segment (start 96.28 67.08) (end 103.45 67.08) (width 0.8) (layer "F.Cu") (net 3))
 (segment (start 110.32 68.9) (end 126.68 68.9) (width 0.8) (layer "F.Cu") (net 4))
 (segment (start 106.68 68.9) (end 108.5 67.08) (width 0.8) (layer "F.Cu") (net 4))
 (segment (start 108.5 67.08) (end 110.32 68.9) (width 0.8) (layer "F.Cu") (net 4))
 (segment (start 88.5 67.08) (end 90.32 68.9) (width 0.8) (layer "F.Cu") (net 4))
 (segment (start 90.32 68.9) (end 106.68 68.9) (width 0.8) (layer "F.Cu") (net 4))
 (segment (start 126.68 68.9) (end 128.5 67.08) (width 0.8) (layer "F.Cu") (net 4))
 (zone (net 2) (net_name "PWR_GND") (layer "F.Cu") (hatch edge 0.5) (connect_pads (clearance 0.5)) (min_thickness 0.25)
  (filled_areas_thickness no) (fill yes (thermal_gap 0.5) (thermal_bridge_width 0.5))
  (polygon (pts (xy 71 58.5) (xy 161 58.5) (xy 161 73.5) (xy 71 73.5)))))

